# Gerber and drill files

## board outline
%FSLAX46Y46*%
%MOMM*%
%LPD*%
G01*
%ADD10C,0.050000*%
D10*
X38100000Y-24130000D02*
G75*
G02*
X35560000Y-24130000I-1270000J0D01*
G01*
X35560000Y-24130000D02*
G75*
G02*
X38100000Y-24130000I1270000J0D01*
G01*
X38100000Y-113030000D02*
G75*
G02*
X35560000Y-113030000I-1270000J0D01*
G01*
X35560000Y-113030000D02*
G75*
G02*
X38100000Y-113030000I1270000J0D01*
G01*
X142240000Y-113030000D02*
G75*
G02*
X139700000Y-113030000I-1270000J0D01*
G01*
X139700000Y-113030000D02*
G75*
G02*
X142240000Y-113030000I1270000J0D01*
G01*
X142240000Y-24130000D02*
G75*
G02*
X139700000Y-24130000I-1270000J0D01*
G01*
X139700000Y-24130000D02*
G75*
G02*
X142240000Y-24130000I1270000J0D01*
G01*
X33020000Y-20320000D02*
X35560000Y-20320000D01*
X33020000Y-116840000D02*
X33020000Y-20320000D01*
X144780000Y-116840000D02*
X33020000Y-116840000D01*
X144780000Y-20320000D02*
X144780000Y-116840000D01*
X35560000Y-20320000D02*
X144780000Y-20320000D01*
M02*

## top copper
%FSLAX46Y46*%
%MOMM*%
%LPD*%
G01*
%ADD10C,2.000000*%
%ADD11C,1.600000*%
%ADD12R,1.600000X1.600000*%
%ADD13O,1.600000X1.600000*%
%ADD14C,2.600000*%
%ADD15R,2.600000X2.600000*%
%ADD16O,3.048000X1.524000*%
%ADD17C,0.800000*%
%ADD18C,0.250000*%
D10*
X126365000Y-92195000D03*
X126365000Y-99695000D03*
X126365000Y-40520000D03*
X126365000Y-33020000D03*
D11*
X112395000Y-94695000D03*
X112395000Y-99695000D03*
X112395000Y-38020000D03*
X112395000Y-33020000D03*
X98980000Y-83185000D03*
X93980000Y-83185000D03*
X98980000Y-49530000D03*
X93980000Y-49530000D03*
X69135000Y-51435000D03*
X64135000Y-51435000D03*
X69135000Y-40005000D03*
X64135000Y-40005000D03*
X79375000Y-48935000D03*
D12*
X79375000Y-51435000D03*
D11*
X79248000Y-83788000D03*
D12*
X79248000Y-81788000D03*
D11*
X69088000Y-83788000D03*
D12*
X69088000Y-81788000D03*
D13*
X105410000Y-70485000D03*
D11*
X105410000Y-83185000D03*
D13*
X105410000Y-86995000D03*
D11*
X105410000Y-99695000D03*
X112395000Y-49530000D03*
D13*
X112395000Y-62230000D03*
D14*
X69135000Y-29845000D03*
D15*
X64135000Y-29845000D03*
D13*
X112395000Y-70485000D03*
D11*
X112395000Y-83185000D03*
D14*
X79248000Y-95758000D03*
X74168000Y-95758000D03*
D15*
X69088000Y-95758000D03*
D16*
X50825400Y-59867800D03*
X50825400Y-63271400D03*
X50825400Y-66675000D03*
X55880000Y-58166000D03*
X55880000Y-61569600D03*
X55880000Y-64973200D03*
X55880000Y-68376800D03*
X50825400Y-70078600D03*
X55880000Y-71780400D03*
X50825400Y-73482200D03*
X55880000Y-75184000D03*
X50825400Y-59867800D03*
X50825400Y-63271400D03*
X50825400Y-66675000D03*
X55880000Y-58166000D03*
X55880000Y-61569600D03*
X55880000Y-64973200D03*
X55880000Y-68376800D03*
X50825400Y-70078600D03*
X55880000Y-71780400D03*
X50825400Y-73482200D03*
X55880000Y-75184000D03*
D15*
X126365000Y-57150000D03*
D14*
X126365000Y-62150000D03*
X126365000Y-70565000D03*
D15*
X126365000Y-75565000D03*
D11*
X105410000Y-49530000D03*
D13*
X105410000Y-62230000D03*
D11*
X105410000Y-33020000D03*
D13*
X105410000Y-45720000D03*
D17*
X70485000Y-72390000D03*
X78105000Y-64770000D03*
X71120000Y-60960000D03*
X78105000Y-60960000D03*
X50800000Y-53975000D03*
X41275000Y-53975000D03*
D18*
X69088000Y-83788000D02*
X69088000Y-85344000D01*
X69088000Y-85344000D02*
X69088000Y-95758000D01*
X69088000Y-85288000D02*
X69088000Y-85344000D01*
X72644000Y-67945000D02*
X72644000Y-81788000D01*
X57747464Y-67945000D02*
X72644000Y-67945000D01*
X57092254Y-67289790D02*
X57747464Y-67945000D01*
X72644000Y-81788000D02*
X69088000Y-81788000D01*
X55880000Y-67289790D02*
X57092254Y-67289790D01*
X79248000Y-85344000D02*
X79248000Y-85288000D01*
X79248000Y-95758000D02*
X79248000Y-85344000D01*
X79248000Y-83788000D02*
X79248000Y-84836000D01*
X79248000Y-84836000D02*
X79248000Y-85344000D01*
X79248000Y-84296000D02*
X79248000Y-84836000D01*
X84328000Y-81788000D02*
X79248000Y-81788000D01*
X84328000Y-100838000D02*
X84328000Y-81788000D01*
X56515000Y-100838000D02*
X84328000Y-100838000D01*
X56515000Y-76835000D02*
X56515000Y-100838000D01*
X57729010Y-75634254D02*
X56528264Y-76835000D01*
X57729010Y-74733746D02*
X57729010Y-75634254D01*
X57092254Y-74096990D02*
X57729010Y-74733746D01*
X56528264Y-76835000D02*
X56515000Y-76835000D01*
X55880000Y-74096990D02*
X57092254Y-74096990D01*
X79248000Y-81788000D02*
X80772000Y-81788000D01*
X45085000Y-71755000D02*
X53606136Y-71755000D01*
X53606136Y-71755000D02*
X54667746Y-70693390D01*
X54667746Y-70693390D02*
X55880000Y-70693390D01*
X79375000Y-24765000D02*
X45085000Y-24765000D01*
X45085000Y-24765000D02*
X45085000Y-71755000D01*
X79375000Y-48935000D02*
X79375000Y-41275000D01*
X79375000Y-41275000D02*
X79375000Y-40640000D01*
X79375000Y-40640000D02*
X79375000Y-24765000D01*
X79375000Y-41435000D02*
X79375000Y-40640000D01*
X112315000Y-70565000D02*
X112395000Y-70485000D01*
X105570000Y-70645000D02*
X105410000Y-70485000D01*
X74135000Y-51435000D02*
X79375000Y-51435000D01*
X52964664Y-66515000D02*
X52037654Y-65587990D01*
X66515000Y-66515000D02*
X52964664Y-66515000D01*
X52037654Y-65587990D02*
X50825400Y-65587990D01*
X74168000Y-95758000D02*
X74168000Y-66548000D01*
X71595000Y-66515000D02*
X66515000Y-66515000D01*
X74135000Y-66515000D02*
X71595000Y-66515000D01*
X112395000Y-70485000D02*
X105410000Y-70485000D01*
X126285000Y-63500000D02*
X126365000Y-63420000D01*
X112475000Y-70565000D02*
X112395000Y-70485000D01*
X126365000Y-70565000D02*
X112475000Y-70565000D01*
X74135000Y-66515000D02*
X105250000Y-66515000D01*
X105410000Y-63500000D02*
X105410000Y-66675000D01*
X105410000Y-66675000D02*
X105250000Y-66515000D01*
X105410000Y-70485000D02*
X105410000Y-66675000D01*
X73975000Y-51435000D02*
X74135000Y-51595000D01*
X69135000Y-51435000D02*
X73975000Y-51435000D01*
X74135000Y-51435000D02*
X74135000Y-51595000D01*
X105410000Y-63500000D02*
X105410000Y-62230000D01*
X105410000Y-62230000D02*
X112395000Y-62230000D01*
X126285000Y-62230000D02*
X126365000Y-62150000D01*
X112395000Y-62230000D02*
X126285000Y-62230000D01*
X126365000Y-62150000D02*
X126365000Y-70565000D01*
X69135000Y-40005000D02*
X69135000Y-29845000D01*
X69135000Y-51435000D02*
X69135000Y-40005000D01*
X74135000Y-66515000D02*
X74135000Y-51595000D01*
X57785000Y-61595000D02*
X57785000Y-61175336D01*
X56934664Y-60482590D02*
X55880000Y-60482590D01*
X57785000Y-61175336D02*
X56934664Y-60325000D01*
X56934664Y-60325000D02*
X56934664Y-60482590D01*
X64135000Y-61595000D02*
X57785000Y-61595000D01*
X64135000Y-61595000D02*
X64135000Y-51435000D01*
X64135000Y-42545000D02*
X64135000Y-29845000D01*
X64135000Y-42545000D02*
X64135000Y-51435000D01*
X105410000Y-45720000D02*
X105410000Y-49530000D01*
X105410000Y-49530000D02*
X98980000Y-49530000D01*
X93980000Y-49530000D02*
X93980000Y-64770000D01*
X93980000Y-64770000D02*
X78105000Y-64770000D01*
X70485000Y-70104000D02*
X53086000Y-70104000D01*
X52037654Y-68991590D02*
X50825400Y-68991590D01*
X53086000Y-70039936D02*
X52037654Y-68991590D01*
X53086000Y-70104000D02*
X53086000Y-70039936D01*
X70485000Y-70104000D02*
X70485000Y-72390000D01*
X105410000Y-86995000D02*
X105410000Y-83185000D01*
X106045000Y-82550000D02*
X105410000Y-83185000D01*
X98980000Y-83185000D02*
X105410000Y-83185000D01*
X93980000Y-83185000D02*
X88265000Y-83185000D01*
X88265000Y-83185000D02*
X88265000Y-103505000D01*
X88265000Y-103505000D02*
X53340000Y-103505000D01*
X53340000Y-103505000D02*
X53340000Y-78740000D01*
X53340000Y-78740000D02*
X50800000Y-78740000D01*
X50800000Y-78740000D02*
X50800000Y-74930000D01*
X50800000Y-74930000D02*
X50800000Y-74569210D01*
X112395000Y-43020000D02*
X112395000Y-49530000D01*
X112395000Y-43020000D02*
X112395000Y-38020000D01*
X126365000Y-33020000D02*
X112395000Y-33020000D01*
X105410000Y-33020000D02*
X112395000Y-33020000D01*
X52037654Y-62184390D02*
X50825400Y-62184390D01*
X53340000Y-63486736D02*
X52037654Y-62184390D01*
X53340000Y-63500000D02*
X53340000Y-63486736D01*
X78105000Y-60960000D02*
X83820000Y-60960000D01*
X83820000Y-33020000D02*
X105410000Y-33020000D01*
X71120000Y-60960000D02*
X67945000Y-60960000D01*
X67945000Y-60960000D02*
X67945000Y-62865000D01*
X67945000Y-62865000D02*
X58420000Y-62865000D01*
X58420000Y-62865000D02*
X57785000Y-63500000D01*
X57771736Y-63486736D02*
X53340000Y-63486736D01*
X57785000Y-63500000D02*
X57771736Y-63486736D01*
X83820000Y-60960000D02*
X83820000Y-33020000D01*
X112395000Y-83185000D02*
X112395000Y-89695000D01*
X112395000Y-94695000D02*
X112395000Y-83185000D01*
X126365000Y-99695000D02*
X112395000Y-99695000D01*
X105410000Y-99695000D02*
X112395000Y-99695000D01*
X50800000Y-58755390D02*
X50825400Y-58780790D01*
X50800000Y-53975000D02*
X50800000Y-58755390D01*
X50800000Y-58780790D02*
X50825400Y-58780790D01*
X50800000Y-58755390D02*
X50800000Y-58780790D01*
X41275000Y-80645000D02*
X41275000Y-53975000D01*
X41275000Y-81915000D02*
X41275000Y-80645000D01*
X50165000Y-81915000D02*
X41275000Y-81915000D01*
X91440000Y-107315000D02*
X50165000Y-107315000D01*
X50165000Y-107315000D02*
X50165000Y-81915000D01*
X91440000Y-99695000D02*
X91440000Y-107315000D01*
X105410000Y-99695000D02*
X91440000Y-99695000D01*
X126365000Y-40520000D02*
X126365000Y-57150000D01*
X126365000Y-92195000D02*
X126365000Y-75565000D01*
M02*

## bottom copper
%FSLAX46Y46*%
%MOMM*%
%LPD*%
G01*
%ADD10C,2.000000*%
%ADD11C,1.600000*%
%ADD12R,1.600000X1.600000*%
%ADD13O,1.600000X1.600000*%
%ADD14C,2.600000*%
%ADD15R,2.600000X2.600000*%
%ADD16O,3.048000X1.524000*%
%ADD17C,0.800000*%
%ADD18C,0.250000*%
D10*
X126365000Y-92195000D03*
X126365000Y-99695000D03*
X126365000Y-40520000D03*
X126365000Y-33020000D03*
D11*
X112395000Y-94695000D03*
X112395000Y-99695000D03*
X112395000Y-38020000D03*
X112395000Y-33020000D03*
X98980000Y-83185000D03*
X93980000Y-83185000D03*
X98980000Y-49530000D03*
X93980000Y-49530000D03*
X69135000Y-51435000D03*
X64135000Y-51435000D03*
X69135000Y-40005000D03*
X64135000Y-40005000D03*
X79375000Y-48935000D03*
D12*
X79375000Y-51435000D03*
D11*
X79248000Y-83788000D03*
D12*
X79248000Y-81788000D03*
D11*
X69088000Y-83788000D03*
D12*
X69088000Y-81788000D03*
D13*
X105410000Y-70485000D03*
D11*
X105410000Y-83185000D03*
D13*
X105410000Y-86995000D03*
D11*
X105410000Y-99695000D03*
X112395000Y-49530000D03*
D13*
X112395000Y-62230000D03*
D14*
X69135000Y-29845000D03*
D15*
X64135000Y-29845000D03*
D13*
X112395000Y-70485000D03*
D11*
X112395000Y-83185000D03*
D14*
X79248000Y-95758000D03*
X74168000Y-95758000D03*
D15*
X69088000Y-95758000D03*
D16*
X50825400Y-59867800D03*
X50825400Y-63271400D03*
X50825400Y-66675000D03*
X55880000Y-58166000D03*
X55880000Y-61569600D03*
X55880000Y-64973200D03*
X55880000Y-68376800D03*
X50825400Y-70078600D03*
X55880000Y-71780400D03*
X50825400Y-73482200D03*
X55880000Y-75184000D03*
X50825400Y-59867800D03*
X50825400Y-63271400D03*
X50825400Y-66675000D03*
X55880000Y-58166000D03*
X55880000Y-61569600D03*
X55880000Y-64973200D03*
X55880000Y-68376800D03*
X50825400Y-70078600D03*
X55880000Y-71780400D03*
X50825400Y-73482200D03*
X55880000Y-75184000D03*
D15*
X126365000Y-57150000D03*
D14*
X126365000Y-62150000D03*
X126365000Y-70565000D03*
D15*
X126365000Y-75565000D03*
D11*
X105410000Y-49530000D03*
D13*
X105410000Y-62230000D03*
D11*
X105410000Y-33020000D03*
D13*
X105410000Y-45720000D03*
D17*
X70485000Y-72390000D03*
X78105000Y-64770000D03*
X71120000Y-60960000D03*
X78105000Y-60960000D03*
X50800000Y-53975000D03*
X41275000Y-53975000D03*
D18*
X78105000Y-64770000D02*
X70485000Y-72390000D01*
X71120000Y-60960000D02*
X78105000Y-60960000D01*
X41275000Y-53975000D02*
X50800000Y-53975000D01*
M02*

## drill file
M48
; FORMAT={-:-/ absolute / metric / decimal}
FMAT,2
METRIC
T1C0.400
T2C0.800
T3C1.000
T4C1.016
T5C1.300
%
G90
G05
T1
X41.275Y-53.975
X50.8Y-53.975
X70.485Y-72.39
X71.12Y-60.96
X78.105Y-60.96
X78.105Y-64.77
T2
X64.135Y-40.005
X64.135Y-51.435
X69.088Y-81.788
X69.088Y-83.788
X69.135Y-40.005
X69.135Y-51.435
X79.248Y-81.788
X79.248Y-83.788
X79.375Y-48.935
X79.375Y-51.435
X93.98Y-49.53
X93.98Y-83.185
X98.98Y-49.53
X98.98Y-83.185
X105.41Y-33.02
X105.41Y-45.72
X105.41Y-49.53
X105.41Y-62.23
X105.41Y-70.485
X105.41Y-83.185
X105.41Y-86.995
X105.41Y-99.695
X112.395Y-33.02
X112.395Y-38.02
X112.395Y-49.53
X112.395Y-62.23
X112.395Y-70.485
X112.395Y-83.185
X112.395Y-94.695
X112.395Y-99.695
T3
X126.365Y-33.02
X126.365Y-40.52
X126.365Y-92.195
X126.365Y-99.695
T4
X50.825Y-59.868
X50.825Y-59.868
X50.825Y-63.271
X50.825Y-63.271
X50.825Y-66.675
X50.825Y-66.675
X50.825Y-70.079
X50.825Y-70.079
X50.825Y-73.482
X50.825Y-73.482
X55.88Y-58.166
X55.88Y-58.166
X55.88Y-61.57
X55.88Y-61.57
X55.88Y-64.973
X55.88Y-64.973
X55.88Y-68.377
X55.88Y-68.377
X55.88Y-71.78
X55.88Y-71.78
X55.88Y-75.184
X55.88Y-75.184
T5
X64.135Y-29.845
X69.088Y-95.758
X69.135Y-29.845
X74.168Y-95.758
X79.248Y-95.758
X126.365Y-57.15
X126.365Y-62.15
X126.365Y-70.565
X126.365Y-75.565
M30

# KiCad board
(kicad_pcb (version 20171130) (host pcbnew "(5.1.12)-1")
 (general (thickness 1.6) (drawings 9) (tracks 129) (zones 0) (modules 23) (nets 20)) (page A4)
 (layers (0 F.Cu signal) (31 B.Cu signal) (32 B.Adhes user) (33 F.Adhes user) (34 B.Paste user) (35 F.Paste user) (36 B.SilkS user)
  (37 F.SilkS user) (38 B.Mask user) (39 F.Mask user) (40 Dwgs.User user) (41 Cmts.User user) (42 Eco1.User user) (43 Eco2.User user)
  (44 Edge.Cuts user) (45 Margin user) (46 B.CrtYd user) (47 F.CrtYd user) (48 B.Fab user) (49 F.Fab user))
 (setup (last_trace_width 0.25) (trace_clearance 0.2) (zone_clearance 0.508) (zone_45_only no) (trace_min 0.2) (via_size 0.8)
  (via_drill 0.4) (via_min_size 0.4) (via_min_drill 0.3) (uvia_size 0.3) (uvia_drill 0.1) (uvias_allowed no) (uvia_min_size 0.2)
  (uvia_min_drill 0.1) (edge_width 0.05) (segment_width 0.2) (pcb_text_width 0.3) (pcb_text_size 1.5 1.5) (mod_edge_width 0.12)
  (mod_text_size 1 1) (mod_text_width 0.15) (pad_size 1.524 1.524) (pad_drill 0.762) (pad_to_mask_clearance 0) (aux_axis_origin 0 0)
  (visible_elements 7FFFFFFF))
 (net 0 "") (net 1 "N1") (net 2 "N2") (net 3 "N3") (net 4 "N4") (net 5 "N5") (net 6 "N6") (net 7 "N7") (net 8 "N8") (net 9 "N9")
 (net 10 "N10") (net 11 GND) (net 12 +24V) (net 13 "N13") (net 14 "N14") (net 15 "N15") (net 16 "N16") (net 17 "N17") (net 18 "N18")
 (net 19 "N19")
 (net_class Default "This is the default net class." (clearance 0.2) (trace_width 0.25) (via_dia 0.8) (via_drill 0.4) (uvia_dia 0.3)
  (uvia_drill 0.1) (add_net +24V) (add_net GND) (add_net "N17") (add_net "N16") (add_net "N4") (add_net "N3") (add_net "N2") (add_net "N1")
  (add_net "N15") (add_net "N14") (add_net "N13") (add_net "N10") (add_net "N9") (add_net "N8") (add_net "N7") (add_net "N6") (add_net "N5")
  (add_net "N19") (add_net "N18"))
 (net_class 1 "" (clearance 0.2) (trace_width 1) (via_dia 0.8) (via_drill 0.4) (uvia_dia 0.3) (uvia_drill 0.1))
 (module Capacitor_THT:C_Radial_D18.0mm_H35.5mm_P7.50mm (layer F.Cu) (at 126.365 99.695 90)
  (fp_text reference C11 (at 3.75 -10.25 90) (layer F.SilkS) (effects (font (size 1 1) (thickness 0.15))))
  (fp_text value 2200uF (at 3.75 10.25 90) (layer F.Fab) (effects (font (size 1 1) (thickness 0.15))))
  (pad 2 thru_hole circle (at 7.5 0 90) (size 2 2) (drill 1) (layers *.Cu *.Mask) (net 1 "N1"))
  (pad 1 thru_hole circle (at 0 0 90) (size 2 2) (drill 1) (layers *.Cu *.Mask) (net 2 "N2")))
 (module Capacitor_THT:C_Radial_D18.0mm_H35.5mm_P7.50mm (layer F.Cu) (at 126.365 33.02 270)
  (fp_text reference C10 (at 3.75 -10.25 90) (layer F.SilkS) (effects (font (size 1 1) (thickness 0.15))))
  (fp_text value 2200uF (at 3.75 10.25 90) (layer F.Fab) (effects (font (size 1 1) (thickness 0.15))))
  (pad 2 thru_hole circle (at 7.5 0 270) (size 2 2) (drill 1) (layers *.Cu *.Mask) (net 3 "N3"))
  (pad 1 thru_hole circle (at 0 0 270) (size 2 2) (drill 1) (layers *.Cu *.Mask) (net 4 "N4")))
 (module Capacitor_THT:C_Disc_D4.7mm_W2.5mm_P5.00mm (layer F.Cu) (at 112.395 99.695 90)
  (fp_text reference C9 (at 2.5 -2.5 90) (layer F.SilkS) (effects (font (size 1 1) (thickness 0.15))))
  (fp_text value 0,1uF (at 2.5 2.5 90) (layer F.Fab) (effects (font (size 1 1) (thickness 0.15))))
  (pad 2 thru_hole circle (at 5 0 90) (size 1.6 1.6) (drill 0.8) (layers *.Cu *.Mask) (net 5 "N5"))
  (pad 1 thru_hole circle (at 0 0 90) (size 1.6 1.6) (drill 0.8) (layers *.Cu *.Mask) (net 2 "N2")))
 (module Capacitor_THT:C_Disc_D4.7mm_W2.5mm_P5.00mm (layer F.Cu) (at 112.395 33.02 270)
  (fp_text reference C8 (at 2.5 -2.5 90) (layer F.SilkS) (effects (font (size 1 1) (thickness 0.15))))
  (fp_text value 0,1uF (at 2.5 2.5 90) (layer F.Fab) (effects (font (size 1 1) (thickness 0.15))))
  (pad 2 thru_hole circle (at 5 0 270) (size 1.6 1.6) (drill 0.8) (layers *.Cu *.Mask) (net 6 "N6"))
  (pad 1 thru_hole circle (at 0 0 270) (size 1.6 1.6) (drill 0.8) (layers *.Cu *.Mask) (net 4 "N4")))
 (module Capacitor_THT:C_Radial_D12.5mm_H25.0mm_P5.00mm (layer F.Cu) (at 93.98 83.185)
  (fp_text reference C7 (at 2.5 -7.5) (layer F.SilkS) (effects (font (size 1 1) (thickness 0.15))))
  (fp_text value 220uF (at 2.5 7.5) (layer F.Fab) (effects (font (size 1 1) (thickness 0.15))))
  (pad 2 thru_hole circle (at 5 0) (size 1.6 1.6) (drill 0.8) (layers *.Cu *.Mask) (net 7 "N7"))
  (pad 1 thru_hole circle (at 0 0) (size 1.6 1.6) (drill 0.8) (layers *.Cu *.Mask) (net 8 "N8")))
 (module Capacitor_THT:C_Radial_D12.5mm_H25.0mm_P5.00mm (layer F.Cu) (at 93.98 49.53)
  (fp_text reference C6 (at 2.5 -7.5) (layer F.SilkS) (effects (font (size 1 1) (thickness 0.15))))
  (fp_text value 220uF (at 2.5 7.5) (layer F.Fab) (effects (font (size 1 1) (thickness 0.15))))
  (pad 2 thru_hole circle (at 5 0) (size 1.6 1.6) (drill 0.8) (layers *.Cu *.Mask) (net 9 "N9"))
  (pad 1 thru_hole circle (at 0 0) (size 1.6 1.6) (drill 0.8) (layers *.Cu *.Mask) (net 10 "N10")))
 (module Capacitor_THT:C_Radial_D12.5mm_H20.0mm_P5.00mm (layer F.Cu) (at 64.135 51.435)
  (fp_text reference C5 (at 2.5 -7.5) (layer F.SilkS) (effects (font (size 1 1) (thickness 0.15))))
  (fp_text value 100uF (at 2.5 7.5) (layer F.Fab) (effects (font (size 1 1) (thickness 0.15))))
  (pad 2 thru_hole circle (at 5 0) (size 1.6 1.6) (drill 0.8) (layers *.Cu *.Mask) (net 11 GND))
  (pad 1 thru_hole circle (at 0 0) (size 1.6 1.6) (drill 0.8) (layers *.Cu *.Mask) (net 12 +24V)))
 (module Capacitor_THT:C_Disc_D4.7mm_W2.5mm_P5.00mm (layer F.Cu) (at 64.135 40.005)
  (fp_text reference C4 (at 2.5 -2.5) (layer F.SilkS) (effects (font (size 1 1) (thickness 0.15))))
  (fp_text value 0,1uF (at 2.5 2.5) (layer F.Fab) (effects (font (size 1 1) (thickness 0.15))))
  (pad 2 thru_hole circle (at 5 0) (size 1.6 1.6) (drill 0.8) (layers *.Cu *.Mask) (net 11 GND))
  (pad 1 thru_hole circle (at 0 0) (size 1.6 1.6) (drill 0.8) (layers *.Cu *.Mask) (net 12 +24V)))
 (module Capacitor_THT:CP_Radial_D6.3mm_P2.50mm (layer F.Cu) (at 79.375 51.435 90)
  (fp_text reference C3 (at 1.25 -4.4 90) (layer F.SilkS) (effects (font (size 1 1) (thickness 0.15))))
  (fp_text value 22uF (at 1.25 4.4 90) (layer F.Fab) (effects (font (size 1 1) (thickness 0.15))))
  (pad 2 thru_hole circle (at 2.5 0 90) (size 1.6 1.6) (drill 0.8) (layers *.Cu *.Mask) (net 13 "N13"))
  (pad 1 thru_hole rect (at 0 0 90) (size 1.6 1.6) (drill 0.8) (layers *.Cu *.Mask) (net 11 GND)))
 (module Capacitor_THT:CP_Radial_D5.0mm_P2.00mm (layer F.Cu) (at 79.248 81.788 270)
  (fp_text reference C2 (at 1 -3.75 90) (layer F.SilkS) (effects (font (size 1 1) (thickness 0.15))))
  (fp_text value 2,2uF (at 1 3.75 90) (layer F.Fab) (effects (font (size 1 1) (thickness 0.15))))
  (pad 2 thru_hole circle (at 2 0 270) (size 1.6 1.6) (drill 0.8) (layers *.Cu *.Mask) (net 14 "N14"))
  (pad 1 thru_hole rect (at 0 0 270) (size 1.6 1.6) (drill 0.8) (layers *.Cu *.Mask) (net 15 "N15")))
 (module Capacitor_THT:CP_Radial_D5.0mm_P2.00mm (layer F.Cu) (at 69.088 81.788 270)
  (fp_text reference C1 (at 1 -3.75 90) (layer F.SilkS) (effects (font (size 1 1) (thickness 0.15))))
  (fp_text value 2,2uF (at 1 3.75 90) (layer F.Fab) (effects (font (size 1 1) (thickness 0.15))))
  (pad 2 thru_hole circle (at 2 0 270) (size 1.6 1.6) (drill 0.8) (layers *.Cu *.Mask) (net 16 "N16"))
  (pad 1 thru_hole rect (at 0 0 270) (size 1.6 1.6) (drill 0.8) (layers *.Cu *.Mask) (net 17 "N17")))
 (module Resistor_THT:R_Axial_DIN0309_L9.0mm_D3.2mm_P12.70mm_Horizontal (layer F.Cu) (at 105.41 83.185 90)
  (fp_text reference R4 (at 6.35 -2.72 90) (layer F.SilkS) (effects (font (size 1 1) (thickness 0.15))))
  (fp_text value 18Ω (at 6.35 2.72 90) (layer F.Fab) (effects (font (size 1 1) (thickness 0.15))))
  (pad 2 thru_hole oval (at 12.7 0 90) (size 1.6 1.6) (drill 0.8) (layers *.Cu *.Mask) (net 11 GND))
  (pad 1 thru_hole circle (at 0 0 90) (size 1.6 1.6) (drill 0.8) (layers *.Cu *.Mask) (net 7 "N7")))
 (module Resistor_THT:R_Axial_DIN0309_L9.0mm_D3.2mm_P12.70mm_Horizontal (layer F.Cu) (at 105.41 99.695 90)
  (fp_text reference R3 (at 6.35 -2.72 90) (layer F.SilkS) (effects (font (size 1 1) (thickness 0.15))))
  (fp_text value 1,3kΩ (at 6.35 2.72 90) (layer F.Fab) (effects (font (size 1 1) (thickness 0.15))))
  (pad 2 thru_hole oval (at 12.7 0 90) (size 1.6 1.6) (drill 0.8) (layers *.Cu *.Mask) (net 7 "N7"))
  (pad 1 thru_hole circle (at 0 0 90) (size 1.6 1.6) (drill 0.8) (layers *.Cu *.Mask) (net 2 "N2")))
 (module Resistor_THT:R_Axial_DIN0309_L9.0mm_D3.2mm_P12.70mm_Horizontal (layer F.Cu) (at 112.395 49.53 270)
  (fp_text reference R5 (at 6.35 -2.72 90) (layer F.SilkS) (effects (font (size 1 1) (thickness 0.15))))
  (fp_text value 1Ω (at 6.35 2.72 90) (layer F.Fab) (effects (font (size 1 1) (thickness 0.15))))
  (pad 1 thru_hole circle (at 0 0 270) (size 1.6 1.6) (drill 0.8) (layers *.Cu *.Mask) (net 6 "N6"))
  (pad 2 thru_hole oval (at 12.7 0 270) (size 1.6 1.6) (drill 0.8) (layers *.Cu *.Mask) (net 11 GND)))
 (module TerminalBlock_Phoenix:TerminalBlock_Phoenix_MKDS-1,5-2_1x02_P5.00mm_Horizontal (layer F.Cu) (at 64.135 29.845)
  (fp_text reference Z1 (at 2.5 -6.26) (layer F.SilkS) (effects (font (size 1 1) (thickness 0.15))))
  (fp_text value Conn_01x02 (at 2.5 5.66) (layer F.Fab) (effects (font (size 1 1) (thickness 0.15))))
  (pad 2 thru_hole circle (at 5 0) (size 2.6 2.6) (drill 1.3) (layers *.Cu *.Mask) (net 11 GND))
  (pad 1 thru_hole rect (at 0 0) (size 2.6 2.6) (drill 1.3) (layers *.Cu *.Mask) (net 12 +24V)))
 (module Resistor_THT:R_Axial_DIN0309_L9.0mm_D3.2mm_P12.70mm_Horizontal (layer F.Cu) (at 112.395 83.185 90)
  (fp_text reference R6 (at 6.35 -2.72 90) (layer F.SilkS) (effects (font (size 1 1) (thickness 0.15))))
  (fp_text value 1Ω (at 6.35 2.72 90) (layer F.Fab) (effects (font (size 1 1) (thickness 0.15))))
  (pad 2 thru_hole oval (at 12.7 0 90) (size 1.6 1.6) (drill 0.8) (layers *.Cu *.Mask) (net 11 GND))
  (pad 1 thru_hole circle (at 0 0 90) (size 1.6 1.6) (drill 0.8) (layers *.Cu *.Mask) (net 5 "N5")))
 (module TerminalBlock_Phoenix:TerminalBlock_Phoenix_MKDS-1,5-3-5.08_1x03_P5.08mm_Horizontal (layer F.Cu) (at 69.088 95.758)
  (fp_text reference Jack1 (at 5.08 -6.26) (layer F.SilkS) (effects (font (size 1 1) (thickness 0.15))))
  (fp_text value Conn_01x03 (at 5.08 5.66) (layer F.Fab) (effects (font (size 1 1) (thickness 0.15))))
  (pad 3 thru_hole circle (at 10.16 0) (size 2.6 2.6) (drill 1.3) (layers *.Cu *.Mask) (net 14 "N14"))
  (pad 2 thru_hole circle (at 5.08 0) (size 2.6 2.6) (drill 1.3) (layers *.Cu *.Mask) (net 11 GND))
  (pad 1 thru_hole rect (at 0 0) (size 2.6 2.6) (drill 1.3) (layers *.Cu *.Mask) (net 16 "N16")))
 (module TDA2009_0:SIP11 (layer F.Cu) (at 46.355 66.675 90)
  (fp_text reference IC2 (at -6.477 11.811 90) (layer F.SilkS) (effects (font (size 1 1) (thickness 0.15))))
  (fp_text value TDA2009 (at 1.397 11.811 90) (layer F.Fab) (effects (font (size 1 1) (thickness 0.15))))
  (pad 10 thru_hole oval (at 6.8072 4.4704 90) (size 1.524 3.048) (drill 1.016) (layers *.Cu *.Mask))
  (pad 8 thru_hole oval (at 3.4036 4.4704 90) (size 1.524 3.048) (drill 1.016) (layers *.Cu *.Mask) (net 4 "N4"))
  (pad 6 thru_hole oval (at 0 4.4704 90) (size 1.524 3.048) (drill 1.016) (layers *.Cu *.Mask))
  (pad 11 thru_hole oval (at 8.509 9.525 90) (size 1.524 3.048) (drill 1.016) (layers *.Cu *.Mask))
  (pad 9 thru_hole oval (at 5.1054 9.525 90) (size 1.524 3.048) (drill 1.016) (layers *.Cu *.Mask))
  (pad 7 thru_hole oval (at 1.7018 9.525 90) (size 1.524 3.048) (drill 1.016) (layers *.Cu *.Mask) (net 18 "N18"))
  (pad 5 thru_hole oval (at -1.7018 9.525 90) (size 1.524 3.048) (drill 1.016) (layers *.Cu *.Mask) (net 17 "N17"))
  (pad 4 thru_hole oval (at -3.4036 4.4704 90) (size 1.524 3.048) (drill 1.016) (layers *.Cu *.Mask) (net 10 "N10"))
  (pad 3 thru_hole oval (at -5.1054 9.525 90) (size 1.524 3.048) (drill 1.016) (layers *.Cu *.Mask))
  (pad 2 thru_hole oval (at -6.8072 4.4704 90) (size 1.524 3.048) (drill 1.016) (layers *.Cu *.Mask))
  (pad 1 thru_hole oval (at -8.509 9.525 90) (size 1.524 3.048) (drill 1.016) (layers *.Cu *.Mask)))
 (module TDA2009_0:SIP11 (layer F.Cu) (at 46.355 66.675 90)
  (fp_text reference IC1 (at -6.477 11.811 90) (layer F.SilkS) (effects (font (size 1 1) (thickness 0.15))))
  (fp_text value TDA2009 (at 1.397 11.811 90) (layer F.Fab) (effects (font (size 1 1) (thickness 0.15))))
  (pad 10 thru_hole oval (at 6.8072 4.4704 90) (size 1.524 3.048) (drill 1.016) (layers *.Cu *.Mask) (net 2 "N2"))
  (pad 8 thru_hole oval (at 3.4036 4.4704 90) (size 1.524 3.048) (drill 1.016) (layers *.Cu *.Mask))
  (pad 6 thru_hole oval (at 0 4.4704 90) (size 1.524 3.048) (drill 1.016) (layers *.Cu *.Mask) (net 11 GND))
  (pad 11 thru_hole oval (at 8.509 9.525 90) (size 1.524 3.048) (drill 1.016) (layers *.Cu *.Mask) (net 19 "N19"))
  (pad 9 thru_hole oval (at 5.1054 9.525 90) (size 1.524 3.048) (drill 1.016) (layers *.Cu *.Mask) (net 12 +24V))
  (pad 7 thru_hole oval (at 1.7018 9.525 90) (size 1.524 3.048) (drill 1.016) (layers *.Cu *.Mask))
  (pad 5 thru_hole oval (at -1.7018 9.525 90) (size 1.524 3.048) (drill 1.016) (layers *.Cu *.Mask))
  (pad 4 thru_hole oval (at -3.4036 4.4704 90) (size 1.524 3.048) (drill 1.016) (layers *.Cu *.Mask))
  (pad 3 thru_hole oval (at -5.1054 9.525 90) (size 1.524 3.048) (drill 1.016) (layers *.Cu *.Mask) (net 13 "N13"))
  (pad 2 thru_hole oval (at -6.8072 4.4704 90) (size 1.524 3.048) (drill 1.016) (layers *.Cu *.Mask) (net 8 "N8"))
  (pad 1 thru_hole oval (at -8.509 9.525 90) (size 1.524 3.048) (drill 1.016) (layers *.Cu *.Mask) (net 15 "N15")))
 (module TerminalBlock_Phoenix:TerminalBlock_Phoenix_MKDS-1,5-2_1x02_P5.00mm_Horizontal (layer F.Cu) (at 126.365 57.15 270)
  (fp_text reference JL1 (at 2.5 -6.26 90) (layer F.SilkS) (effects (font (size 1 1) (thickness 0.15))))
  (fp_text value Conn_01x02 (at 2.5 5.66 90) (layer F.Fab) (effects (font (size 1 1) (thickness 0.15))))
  (pad 1 thru_hole rect (at 0 0 270) (size 2.6 2.6) (drill 1.3) (layers *.Cu *.Mask) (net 3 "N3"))
  (pad 2 thru_hole circle (at 5 0 270) (size 2.6 2.6) (drill 1.3) (layers *.Cu *.Mask) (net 11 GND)))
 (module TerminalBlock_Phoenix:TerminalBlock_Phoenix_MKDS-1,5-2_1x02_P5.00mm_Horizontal (layer F.Cu) (at 126.365 75.565 90)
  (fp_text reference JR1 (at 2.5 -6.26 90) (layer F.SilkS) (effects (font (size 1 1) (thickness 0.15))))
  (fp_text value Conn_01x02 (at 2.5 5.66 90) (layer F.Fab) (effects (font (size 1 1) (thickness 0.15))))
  (pad 2 thru_hole circle (at 5 0 90) (size 2.6 2.6) (drill 1.3) (layers *.Cu *.Mask) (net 11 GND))
  (pad 1 thru_hole rect (at 0 0 90) (size 2.6 2.6) (drill 1.3) (layers *.Cu *.Mask) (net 1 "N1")))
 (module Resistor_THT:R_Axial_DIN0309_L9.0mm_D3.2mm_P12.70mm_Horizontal (layer F.Cu) (at 105.41 49.53 270)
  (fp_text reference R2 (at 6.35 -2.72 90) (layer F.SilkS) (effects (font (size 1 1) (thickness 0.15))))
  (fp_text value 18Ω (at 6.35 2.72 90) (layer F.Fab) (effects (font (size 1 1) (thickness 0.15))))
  (pad 1 thru_hole circle (at 0 0 270) (size 1.6 1.6) (drill 0.8) (layers *.Cu *.Mask) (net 9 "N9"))
  (pad 2 thru_hole oval (at 12.7 0 270) (size 1.6 1.6) (drill 0.8) (layers *.Cu *.Mask) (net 11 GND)))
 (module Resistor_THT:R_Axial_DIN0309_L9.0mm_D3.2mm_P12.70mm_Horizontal (layer F.Cu) (at 105.41 33.02 270)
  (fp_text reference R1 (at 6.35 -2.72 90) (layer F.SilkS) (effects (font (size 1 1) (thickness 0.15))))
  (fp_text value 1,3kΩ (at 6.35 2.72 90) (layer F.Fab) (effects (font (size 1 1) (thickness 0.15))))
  (pad 1 thru_hole circle (at 0 0 270) (size 1.6 1.6) (drill 0.8) (layers *.Cu *.Mask) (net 4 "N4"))
  (pad 2 thru_hole oval (at 12.7 0 270) (size 1.6 1.6) (drill 0.8) (layers *.Cu *.Mask) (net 9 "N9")))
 (gr_circle (center 36.83 24.13) (end 36.83 22.86) (layer Edge.Cuts) (width 0.05))
 (gr_circle (center 36.83 113.03) (end 38.1 113.03) (layer Edge.Cuts) (width 0.05))
 (gr_circle (center 140.97 113.03) (end 142.24 113.03) (layer Edge.Cuts) (width 0.05))
 (gr_circle (center 140.97 24.13) (end 142.24 24.13) (layer Edge.Cuts) (width 0.05))
 (gr_line (start 33.02 20.32) (end 35.56 20.32) (layer Edge.Cuts) (width 0.05))
 (gr_line (start 33.02 116.84) (end 33.02 20.32) (layer Edge.Cuts) (width 0.05))
 (gr_line (start 144.78 116.84) (end 33.02 116.84) (layer Edge.Cuts) (width 0.05))
 (gr_line (start 144.78 20.32) (end 144.78 116.84) (layer Edge.Cuts) (width 0.05))
 (gr_line (start 35.56 20.32) (end 144.78 20.32) (layer Edge.Cuts) (width 0.05))
 (segment (start 69.088 83.788) (end 69.088 85.344) (width 0.25) (layer F.Cu) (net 16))
 (segment (start 69.088 85.344) (end 69.088 95.758) (width 0.25) (layer F.Cu) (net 16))
 (segment (start 69.088 85.288) (end 69.088 85.344) (width 0.25) (layer F.Cu) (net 16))
 (segment (start 72.644 67.945) (end 72.644 81.788) (width 0.25) (layer F.Cu) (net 17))
 (segment (start 57.747464 67.945) (end 72.644 67.945) (width 0.25) (layer F.Cu) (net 17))
 (segment (start 57.092254 67.28979) (end 57.747464 67.945) (width 0.25) (layer F.Cu) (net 17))
 (segment (start 72.644 81.788) (end 69.088 81.788) (width 0.25) (layer F.Cu) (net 17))
 (segment (start 55.88 67.28979) (end 57.092254 67.28979) (width 0.25) (layer F.Cu) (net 17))
 (segment (start 79.248 85.344) (end 79.248 85.288) (width 0.25) (layer F.Cu) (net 14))
 (segment (start 79.248 95.758) (end 79.248 85.344) (width 0.25) (layer F.Cu) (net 14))
 (segment (start 79.248 83.788) (end 79.248 84.836) (width 0.25) (layer F.Cu) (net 14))
 (segment (start 79.248 84.836) (end 79.248 85.344) (width 0.25) (layer F.Cu) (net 14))
 (segment (start 79.248 84.296) (end 79.248 84.836) (width 0.25) (layer F.Cu) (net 14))
 (segment (start 84.328 81.788) (end 79.248 81.788) (width 0.25) (layer F.Cu) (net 15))
 (segment (start 84.328 100.838) (end 84.328 81.788) (width 0.25) (layer F.Cu) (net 15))
 (segment (start 56.515 100.838) (end 84.328 100.838) (width 0.25) (layer F.Cu) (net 15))
 (segment (start 56.515 76.835) (end 56.515 100.838) (width 0.25) (layer F.Cu) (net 15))
 (segment (start 57.72901 75.634254) (end 56.528264 76.835) (width 0.25) (layer F.Cu) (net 15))
 (segment (start 57.72901 74.733746) (end 57.72901 75.634254) (width 0.25) (layer F.Cu) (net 15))
 (segment (start 57.092254 74.09699) (end 57.72901 74.733746) (width 0.25) (layer F.Cu) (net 15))
 (segment (start 56.528264 76.835) (end 56.515 76.835) (width 0.25) (layer F.Cu) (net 15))
 (segment (start 55.88 74.09699) (end 57.092254 74.09699) (width 0.25) (layer F.Cu) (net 15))
 (segment (start 79.248 81.788) (end 80.772 81.788) (width 0.25) (layer F.Cu) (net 15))
 (segment (start 45.085 71.755) (end 53.606136 71.755) (width 0.25) (layer F.Cu) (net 13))
 (segment (start 53.606136 71.755) (end 54.667746 70.69339) (width 0.25) (layer F.Cu) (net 13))
 (segment (start 54.667746 70.69339) (end 55.88 70.69339) (width 0.25) (layer F.Cu) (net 13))
 (segment (start 79.375 24.765) (end 45.085 24.765) (width 0.25) (layer F.Cu) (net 13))
 (segment (start 45.085 24.765) (end 45.085 71.755) (width 0.25) (layer F.Cu) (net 13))
 (segment (start 79.375 48.935) (end 79.375 41.275) (width 0.25) (layer F.Cu) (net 13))
 (segment (start 79.375 41.275) (end 79.375 40.64) (width 0.25) (layer F.Cu) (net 13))
 (segment (start 79.375 40.64) (end 79.375 24.765) (width 0.25) (layer F.Cu) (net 13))
 (segment (start 79.375 41.435) (end 79.375 40.64) (width 0.25) (layer F.Cu) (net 13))
 (segment (start 112.315 70.565) (end 112.395 70.485) (width 0.25) (layer F.Cu) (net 11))
 (segment (start 105.57 70.645) (end 105.41 70.485) (width 0.25) (layer F.Cu) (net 11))
 (segment (start 74.135 51.435) (end 79.375 51.435) (width 0.25) (layer F.Cu) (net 11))
 (segment (start 52.964664 66.515) (end 52.037654 65.58799) (width 0.25) (layer F.Cu) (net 11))
 (segment (start 66.515 66.515) (end 52.964664 66.515) (width 0.25) (layer F.Cu) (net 11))
 (segment (start 52.037654 65.58799) (end 50.8254 65.58799) (width 0.25) (layer F.Cu) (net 11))
 (segment (start 74.168 95.758) (end 74.168 66.548) (width 0.25) (layer F.Cu) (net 11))
 (segment (start 71.595 66.515) (end 66.515 66.515) (width 0.25) (layer F.Cu) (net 11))
 (segment (start 74.135 66.515) (end 71.595 66.515) (width 0.25) (layer F.Cu) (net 11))
 (segment (start 112.395 70.485) (end 105.41 70.485) (width 0.25) (layer F.Cu) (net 11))
 (segment (start 126.285 63.5) (end 126.365 63.42) (width 0.25) (layer F.Cu) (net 11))
 (segment (start 112.475 70.565) (end 112.395 70.485) (width 0.25) (layer F.Cu) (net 11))
 (segment (start 126.365 70.565) (end 112.475 70.565) (width 0.25) (layer F.Cu) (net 11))
 (segment (start 74.135 66.515) (end 105.25 66.515) (width 0.25) (layer F.Cu) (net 11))
 (segment (start 105.41 63.5) (end 105.41 66.675) (width 0.25) (layer F.Cu) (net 11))
 (segment (start 105.41 66.675) (end 105.25 66.515) (width 0.25) (layer F.Cu) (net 11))
 (segment (start 105.41 70.485) (end 105.41 66.675) (width 0.25) (layer F.Cu) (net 11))
 (segment (start 73.975 51.435) (end 74.135 51.595) (width 0.25) (layer F.Cu) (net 11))
 (segment (start 69.135 51.435) (end 73.975 51.435) (width 0.25) (layer F.Cu) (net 11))
 (segment (start 74.135 51.435) (end 74.135 51.595) (width 0.25) (layer F.Cu) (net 11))
 (segment (start 105.41 63.5) (end 105.41 62.23) (width 0.25) (layer F.Cu) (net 11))
 (segment (start 105.41 62.23) (end 112.395 62.23) (width 0.25) (layer F.Cu) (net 11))
 (segment (start 126.285 62.23) (end 126.365 62.15) (width 0.25) (layer F.Cu) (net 11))
 (segment (start 112.395 62.23) (end 126.285 62.23) (width 0.25) (layer F.Cu) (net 11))
 (segment (start 126.365 62.15) (end 126.365 70.565) (width 0.25) (layer F.Cu) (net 11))
 (segment (start 69.135 40.005) (end 69.135 29.845) (width 0.25) (layer F.Cu) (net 11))
 (segment (start 69.135 51.435) (end 69.135 40.005) (width 0.25) (layer F.Cu) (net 11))
 (segment (start 74.135 66.515) (end 74.135 51.595) (width 0.25) (layer F.Cu) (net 11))
 (segment (start 57.785 61.595) (end 57.785 61.175336) (width 0.25) (layer F.Cu) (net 12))
 (segment (start 56.934664 60.48259) (end 55.88 60.48259) (width 0.25) (layer F.Cu) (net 12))
 (segment (start 57.785 61.175336) (end 56.934664 60.325) (width 0.25) (layer F.Cu) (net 12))
 (segment (start 56.934664 60.325) (end 56.934664 60.48259) (width 0.25) (layer F.Cu) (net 12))
 (segment (start 64.135 61.595) (end 57.785 61.595) (width 0.25) (layer F.Cu) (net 12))
 (segment (start 64.135 61.595) (end 64.135 51.435) (width 0.25) (layer F.Cu) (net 12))
 (segment (start 64.135 42.545) (end 64.135 29.845) (width 0.25) (layer F.Cu) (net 12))
 (segment (start 64.135 42.545) (end 64.135 51.435) (width 0.25) (layer F.Cu) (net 12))
 (segment (start 105.41 45.72) (end 105.41 49.53) (width 0.25) (layer F.Cu) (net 9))
 (segment (start 105.41 49.53) (end 98.98 49.53) (width 0.25) (layer F.Cu) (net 9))
 (via (at 70.485 72.39) (size 0.8) (drill 0.4) (layers F.Cu B.Cu) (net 10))
 (via (at 78.105 64.77) (size 0.8) (drill 0.4) (layers F.Cu B.Cu) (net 10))
 (segment (start 93.98 49.53) (end 93.98 64.77) (width 0.25) (layer F.Cu) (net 10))
 (segment (start 93.98 64.77) (end 78.105 64.77) (width 0.25) (layer F.Cu) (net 10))
 (segment (start 70.485 70.104) (end 53.086 70.104) (width 0.25) (layer F.Cu) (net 10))
 (segment (start 52.037654 68.99159) (end 50.8254 68.99159) (width 0.25) (layer F.Cu) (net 10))
 (segment (start 53.086 70.039936) (end 52.037654 68.99159) (width 0.25) (layer F.Cu) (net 10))
 (segment (start 53.086 70.104) (end 53.086 70.039936) (width 0.25) (layer F.Cu) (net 10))
 (segment (start 78.105 64.77) (end 70.485 72.39) (width 0.25) (layer B.Cu) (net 10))
 (segment (start 70.485 70.104) (end 70.485 72.39) (width 0.25) (layer F.Cu) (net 10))
 (segment (start 105.41 86.995) (end 105.41 83.185) (width 0.25) (layer F.Cu) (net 7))
 (segment (start 106.045 82.55) (end 105.41 83.185) (width 0.25) (layer F.Cu) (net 7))
 (segment (start 98.98 83.185) (end 105.41 83.185) (width 0.25) (layer F.Cu) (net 7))
 (segment (start 93.98 83.185) (end 88.265 83.185) (width 0.25) (layer F.Cu) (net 8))
 (segment (start 88.265 83.185) (end 88.265 103.505) (width 0.25) (layer F.Cu) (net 8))
 (segment (start 88.265 103.505) (end 53.34 103.505) (width 0.25) (layer F.Cu) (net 8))
 (segment (start 53.34 103.505) (end 53.34 78.74) (width 0.25) (layer F.Cu) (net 8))
 (segment (start 53.34 78.74) (end 50.8 78.74) (width 0.25) (layer F.Cu) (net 8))
 (segment (start 50.8 78.74) (end 50.8 74.93) (width 0.25) (layer F.Cu) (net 8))
 (segment (start 50.8 74.93) (end 50.8 74.56921) (width 0.25) (layer F.Cu) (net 8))
 (segment (start 112.395 43.02) (end 112.395 49.53) (width 0.25) (layer F.Cu) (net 6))
 (segment (start 112.395 43.02) (end 112.395 38.02) (width 0.25) (layer F.Cu) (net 6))
 (via (at 71.12 60.96) (size 0.8) (drill 0.4) (layers F.Cu B.Cu) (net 4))
 (via (at 78.105 60.96) (size 0.8) (drill 0.4) (layers F.Cu B.Cu) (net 4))
 (segment (start 126.365 33.02) (end 112.395 33.02) (width 0.25) (layer F.Cu) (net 4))
 (segment (start 105.41 33.02) (end 112.395 33.02) (width 0.25) (layer F.Cu) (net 4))
 (segment (start 52.037654 62.18439) (end 50.8254 62.18439) (width 0.25) (layer F.Cu) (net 4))
 (segment (start 53.34 63.486736) (end 52.037654 62.18439) (width 0.25) (layer F.Cu) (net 4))
 (segment (start 53.34 63.5) (end 53.34 63.486736) (width 0.25) (layer F.Cu) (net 4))
 (segment (start 78.105 60.96) (end 83.82 60.96) (width 0.25) (layer F.Cu) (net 4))
 (segment (start 83.82 33.02) (end 105.41 33.02) (width 0.25) (layer F.Cu) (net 4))
 (segment (start 71.12 60.96) (end 78.105 60.96) (width 0.25) (layer B.Cu) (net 4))
 (segment (start 71.12 60.96) (end 67.945 60.96) (width 0.25) (layer F.Cu) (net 4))
 (segment (start 67.945 60.96) (end 67.945 62.865) (width 0.25) (layer F.Cu) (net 4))
 (segment (start 67.945 62.865) (end 58.42 62.865) (width 0.25) (layer F.Cu) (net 4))
 (segment (start 58.42 62.865) (end 57.785 63.5) (width 0.25) (layer F.Cu) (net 4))
 (segment (start 57.771736 63.486736) (end 53.34 63.486736) (width 0.25) (layer F.Cu) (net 4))
 (segment (start 57.785 63.5) (end 57.771736 63.486736) (width 0.25) (layer F.Cu) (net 4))
 (segment (start 83.82 60.96) (end 83.82 33.02) (width 0.25) (layer F.Cu) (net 4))
 (segment (start 112.395 83.185) (end 112.395 89.695) (width 0.25) (layer F.Cu) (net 5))
 (segment (start 112.395 94.695) (end 112.395 83.185) (width 0.25) (layer F.Cu) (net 5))
 (via (at 50.8 53.975) (size 0.8) (drill 0.4) (layers F.Cu B.Cu) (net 2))
 (via (at 41.275 53.975) (size 0.8) (drill 0.4) (layers F.Cu B.Cu) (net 2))
 (segment (start 126.365 99.695) (end 112.395 99.695) (width 0.25) (layer F.Cu) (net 2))
 (segment (start 105.41 99.695) (end 112.395 99.695) (width 0.25) (layer F.Cu) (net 2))
 (segment (start 50.8 58.75539) (end 50.8254 58.78079) (width 0.25) (layer F.Cu) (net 2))
 (segment (start 50.8 53.975) (end 50.8 58.75539) (width 0.25) (layer F.Cu) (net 2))
 (segment (start 50.8 58.78079) (end 50.8254 58.78079) (width 0.25) (layer F.Cu) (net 2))
 (segment (start 50.8 58.75539) (end 50.8 58.78079) (width 0.25) (layer F.Cu) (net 2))
 (segment (start 41.275 53.975) (end 50.8 53.975) (width 0.25) (layer B.Cu) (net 2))
 (segment (start 41.275 80.645) (end 41.275 53.975) (width 0.25) (layer F.Cu) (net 2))
 (segment (start 41.275 81.915) (end 41.275 80.645) (width 0.25) (layer F.Cu) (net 2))
 (segment (start 50.165 81.915) (end 41.275 81.915) (width 0.25) (layer F.Cu) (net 2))
 (segment (start 91.44 107.315) (end 50.165 107.315) (width 0.25) (layer F.Cu) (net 2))
 (segment (start 50.165 107.315) (end 50.165 81.915) (width 0.25) (layer F.Cu) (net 2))
 (segment (start 91.44 99.695) (end 91.44 107.315) (width 0.25) (layer F.Cu) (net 2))
 (segment (start 105.41 99.695) (end 91.44 99.695) (width 0.25) (layer F.Cu) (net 2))
 (segment (start 126.365 40.52) (end 126.365 57.15) (width 0.25) (layer F.Cu) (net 3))
 (segment (start 126.365 92.195) (end 126.365 75.565) (width 0.25) (layer F.Cu) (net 1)))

